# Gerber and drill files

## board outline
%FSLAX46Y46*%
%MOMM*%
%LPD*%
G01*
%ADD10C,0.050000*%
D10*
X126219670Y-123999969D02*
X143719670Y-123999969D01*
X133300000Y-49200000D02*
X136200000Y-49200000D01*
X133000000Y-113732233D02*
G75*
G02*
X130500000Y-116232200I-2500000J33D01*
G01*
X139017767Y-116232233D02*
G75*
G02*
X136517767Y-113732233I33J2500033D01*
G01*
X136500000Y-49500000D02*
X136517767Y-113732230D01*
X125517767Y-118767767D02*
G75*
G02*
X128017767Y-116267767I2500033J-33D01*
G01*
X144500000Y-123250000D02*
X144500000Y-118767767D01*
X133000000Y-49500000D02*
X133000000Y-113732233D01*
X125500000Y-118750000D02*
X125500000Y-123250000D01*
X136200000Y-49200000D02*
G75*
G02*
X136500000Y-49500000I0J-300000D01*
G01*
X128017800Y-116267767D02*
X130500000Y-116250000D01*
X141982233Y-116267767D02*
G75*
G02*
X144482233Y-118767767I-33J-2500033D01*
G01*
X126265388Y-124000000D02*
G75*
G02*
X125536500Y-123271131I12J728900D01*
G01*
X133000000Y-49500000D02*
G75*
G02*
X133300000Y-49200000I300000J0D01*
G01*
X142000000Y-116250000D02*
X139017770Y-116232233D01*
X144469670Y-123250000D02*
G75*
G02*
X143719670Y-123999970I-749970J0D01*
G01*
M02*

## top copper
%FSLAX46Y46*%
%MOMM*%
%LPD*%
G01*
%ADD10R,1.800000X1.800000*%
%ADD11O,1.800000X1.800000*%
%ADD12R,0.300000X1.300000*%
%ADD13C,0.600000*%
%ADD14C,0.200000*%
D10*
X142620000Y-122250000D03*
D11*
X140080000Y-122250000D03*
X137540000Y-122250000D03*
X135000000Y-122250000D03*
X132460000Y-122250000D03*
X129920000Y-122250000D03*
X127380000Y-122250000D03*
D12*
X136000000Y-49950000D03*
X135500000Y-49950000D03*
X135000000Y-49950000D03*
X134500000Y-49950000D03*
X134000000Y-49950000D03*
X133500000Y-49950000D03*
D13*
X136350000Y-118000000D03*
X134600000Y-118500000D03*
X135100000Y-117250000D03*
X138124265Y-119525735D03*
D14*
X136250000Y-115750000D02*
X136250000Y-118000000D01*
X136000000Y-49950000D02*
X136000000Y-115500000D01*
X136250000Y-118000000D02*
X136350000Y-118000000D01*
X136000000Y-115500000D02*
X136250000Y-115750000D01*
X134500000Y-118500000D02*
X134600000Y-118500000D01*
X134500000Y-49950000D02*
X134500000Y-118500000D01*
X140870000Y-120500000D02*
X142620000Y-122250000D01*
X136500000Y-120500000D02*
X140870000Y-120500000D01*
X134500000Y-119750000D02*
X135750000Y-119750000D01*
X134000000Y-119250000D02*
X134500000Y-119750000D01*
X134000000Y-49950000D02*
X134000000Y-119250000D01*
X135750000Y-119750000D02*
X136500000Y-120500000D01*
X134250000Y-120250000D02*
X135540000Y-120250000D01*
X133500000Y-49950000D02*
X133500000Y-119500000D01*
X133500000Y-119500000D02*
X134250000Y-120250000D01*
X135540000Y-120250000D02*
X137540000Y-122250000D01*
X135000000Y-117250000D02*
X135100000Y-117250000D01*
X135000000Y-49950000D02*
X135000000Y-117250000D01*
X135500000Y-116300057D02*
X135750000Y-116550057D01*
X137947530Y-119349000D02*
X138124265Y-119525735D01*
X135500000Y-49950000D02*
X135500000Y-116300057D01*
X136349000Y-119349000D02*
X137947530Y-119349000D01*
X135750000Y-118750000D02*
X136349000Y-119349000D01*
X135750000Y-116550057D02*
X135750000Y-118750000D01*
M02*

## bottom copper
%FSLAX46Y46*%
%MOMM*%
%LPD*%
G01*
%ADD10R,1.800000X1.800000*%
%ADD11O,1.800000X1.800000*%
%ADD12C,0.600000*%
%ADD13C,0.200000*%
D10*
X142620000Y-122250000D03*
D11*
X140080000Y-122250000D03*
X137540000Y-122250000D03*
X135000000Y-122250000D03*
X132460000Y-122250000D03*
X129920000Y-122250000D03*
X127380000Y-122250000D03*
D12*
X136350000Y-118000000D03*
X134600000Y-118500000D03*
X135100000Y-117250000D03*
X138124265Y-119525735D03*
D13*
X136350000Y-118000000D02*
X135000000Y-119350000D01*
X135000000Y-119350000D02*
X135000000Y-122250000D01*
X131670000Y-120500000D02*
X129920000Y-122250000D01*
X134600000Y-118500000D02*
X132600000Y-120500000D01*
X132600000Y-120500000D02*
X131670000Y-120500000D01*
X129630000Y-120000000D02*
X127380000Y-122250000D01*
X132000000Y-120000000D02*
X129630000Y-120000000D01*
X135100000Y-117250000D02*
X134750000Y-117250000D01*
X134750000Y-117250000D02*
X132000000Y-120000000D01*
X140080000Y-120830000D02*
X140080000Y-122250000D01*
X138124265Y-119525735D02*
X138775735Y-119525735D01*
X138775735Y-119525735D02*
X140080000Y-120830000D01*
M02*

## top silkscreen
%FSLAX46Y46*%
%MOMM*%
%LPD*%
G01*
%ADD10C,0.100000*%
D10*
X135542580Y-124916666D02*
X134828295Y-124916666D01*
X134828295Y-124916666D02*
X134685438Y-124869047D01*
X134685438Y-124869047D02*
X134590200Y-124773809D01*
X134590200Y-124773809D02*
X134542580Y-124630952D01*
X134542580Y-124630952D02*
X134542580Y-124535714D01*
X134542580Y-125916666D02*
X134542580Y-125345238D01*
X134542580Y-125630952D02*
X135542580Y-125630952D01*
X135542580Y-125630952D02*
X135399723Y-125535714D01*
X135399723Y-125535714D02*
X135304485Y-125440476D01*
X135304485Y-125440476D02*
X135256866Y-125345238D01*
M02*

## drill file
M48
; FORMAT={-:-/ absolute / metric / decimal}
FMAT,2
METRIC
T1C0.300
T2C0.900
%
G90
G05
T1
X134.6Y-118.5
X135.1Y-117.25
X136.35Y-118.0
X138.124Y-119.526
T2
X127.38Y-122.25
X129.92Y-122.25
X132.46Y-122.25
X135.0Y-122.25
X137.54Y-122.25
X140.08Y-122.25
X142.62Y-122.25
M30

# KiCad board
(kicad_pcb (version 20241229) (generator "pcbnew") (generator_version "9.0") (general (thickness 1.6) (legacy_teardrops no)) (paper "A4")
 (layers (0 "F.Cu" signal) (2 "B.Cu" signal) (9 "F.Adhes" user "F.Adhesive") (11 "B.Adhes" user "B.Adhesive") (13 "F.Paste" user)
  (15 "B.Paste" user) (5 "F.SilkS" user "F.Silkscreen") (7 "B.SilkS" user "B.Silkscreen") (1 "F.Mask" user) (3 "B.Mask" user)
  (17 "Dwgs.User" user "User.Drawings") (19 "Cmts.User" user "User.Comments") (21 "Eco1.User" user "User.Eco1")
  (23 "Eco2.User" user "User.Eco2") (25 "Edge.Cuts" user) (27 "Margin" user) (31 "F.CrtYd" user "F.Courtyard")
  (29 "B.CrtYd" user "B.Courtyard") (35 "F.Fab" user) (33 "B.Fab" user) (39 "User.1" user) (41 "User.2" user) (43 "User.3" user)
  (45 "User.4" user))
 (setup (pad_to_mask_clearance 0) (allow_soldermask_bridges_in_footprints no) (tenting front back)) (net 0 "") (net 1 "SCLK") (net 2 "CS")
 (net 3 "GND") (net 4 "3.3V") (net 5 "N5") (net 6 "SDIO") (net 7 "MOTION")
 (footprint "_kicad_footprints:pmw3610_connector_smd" (layer "F.Cu") (at 135 122.25 -90)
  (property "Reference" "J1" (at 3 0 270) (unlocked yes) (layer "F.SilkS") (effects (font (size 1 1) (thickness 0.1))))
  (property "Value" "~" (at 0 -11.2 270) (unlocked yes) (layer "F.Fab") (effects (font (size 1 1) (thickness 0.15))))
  (pad "1" thru_hole rect (at 0 -7.62 270) (size 1.8 1.8) (drill 0.9) (layers "*.Cu" "*.Mask") (remove_unused_layers no) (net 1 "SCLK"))
  (pad "2" thru_hole oval (at 0 -5.08 270) (size 1.8 1.8) (drill 0.9) (layers "*.Cu" "*.Mask") (remove_unused_layers no) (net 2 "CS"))
  (pad "3" thru_hole oval (at 0 -2.54 270) (size 1.8 1.8) (drill 0.9) (layers "*.Cu" "*.Mask") (remove_unused_layers no) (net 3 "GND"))
  (pad "4" thru_hole oval (at 0 0 270) (size 1.8 1.8) (drill 0.9) (layers "*.Cu" "*.Mask") (remove_unused_layers no) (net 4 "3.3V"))
  (pad "5" thru_hole oval (at 0 2.54 270) (size 1.8 1.8) (drill 0.9) (layers "*.Cu" "*.Mask") (remove_unused_layers no) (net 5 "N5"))
  (pad "6" thru_hole oval (at 0 5.08 270) (size 1.8 1.8) (drill 0.9) (layers "*.Cu" "*.Mask") (remove_unused_layers no) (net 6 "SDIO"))
  (pad "7" thru_hole oval (at 0 7.62 270) (size 1.8 1.8) (drill 0.9) (layers "*.Cu" "*.Mask") (remove_unused_layers no) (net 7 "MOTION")))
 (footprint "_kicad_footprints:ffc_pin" (layer "B.Cu") (at 134.5 45.95)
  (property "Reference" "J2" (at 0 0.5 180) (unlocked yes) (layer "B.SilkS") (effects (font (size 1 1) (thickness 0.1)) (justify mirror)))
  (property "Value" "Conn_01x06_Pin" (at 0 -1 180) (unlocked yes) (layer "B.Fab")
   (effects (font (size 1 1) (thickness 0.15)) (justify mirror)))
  (pad "1" smd rect (at 1.5 4) (size 0.3 1.3) (layers "F.Cu" "F.Mask" "F.Paste") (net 4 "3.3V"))
  (pad "2" smd rect (at 1 4) (size 0.3 1.3) (layers "F.Cu" "F.Mask" "F.Paste") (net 2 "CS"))
  (pad "3" smd rect (at 0.5 4) (size 0.3 1.3) (layers "F.Cu" "F.Mask" "F.Paste") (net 7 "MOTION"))
  (pad "4" smd rect (at 0 4) (size 0.3 1.3) (layers "F.Cu" "F.Mask" "F.Paste") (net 6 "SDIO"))
  (pad "5" smd rect (at -0.5 4) (size 0.3 1.3) (layers "F.Cu" "F.Mask" "F.Paste") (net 1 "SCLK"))
  (pad "6" smd rect (at -1 4) (size 0.3 1.3) (layers "F.Cu" "F.Mask" "F.Paste") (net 3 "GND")))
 (gr_line (start 126.21967 123.999969) (end 143.71967 123.999969) (stroke (width 0.05) (type default)) (layer "Edge.Cuts"))
 (gr_line (start 133.3 49.2) (end 136.2 49.2) (stroke (width 0.05) (type default)) (layer "Edge.Cuts"))
 (gr_arc (start 133 113.732233) (mid 132.267767 115.5) (end 130.5 116.232233) (stroke (width 0.05) (type default)) (layer "Edge.Cuts"))
 (gr_arc (start 139.017767 116.232233) (mid 137.25 115.5) (end 136.517767 113.732233) (stroke (width 0.05) (type default))
  (layer "Edge.Cuts"))
 (gr_line (start 136.5 49.5) (end 136.517767 113.73223) (stroke (width 0.05) (type default)) (layer "Edge.Cuts"))
 (gr_arc (start 125.517767 118.767767) (mid 126.25 117) (end 128.017767 116.267767) (stroke (width 0.05) (type default)) (layer "Edge.Cuts"))
 (gr_line (start 144.5 123.25) (end 144.5 118.767767) (stroke (width 0.05) (type default)) (layer "Edge.Cuts"))
 (gr_line (start 133 49.5) (end 133 113.732233) (stroke (width 0.05) (type default)) (layer "Edge.Cuts"))
 (gr_line (start 125.5 118.75) (end 125.5 123.25) (stroke (width 0.05) (type default)) (layer "Edge.Cuts"))
 (gr_arc (start 136.2 49.2) (mid 136.412132 49.287868) (end 136.5 49.5) (stroke (width 0.05) (type default)) (layer "Edge.Cuts"))
 (gr_line (start 128.0178 116.267767) (end 130.5 116.25) (stroke (width 0.05) (type default)) (layer "Edge.Cuts"))
 (gr_arc (start 141.982233 116.267767) (mid 143.75 117) (end 144.482233 118.767767) (stroke (width 0.05) (type default)) (layer "Edge.Cuts"))
 (gr_arc (start 126.265388 124) (mid 125.75 123.786519) (end 125.536519 123.271131) (stroke (width 0.05) (type default)) (layer "Edge.Cuts"))
 (gr_arc (start 133 49.5) (mid 133.087868 49.287868) (end 133.3 49.2) (stroke (width 0.05) (type default)) (layer "Edge.Cuts"))
 (gr_line (start 142 116.25) (end 139.01777 116.232233) (stroke (width 0.05) (type default)) (layer "Edge.Cuts"))
 (gr_arc (start 144.46967 123.25) (mid 144.25 123.78033) (end 143.71967 124) (stroke (width 0.05) (type default)) (layer "Edge.Cuts"))
 (segment (start 136.25 115.75) (end 136.25 118) (width 0.2) (layer "F.Cu") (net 4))
 (segment (start 136 49.95) (end 136 115.5) (width 0.2) (layer "F.Cu") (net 4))
 (segment (start 136.25 118) (end 136.35 118) (width 0.2) (layer "F.Cu") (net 4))
 (segment (start 136 115.5) (end 136.25 115.75) (width 0.2) (layer "F.Cu") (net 4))
 (via (at 136.35 118) (size 0.6) (drill 0.3) (layers "F.Cu" "B.Cu") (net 4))
 (segment (start 136.35 118) (end 135 119.35) (width 0.2) (layer "B.Cu") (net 4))
 (segment (start 135 119.35) (end 135 122.25) (width 0.2) (layer "B.Cu") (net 4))
 (segment (start 134.5 118.5) (end 134.6 118.5) (width 0.2) (layer "F.Cu") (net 6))
 (segment (start 134.5 49.95) (end 134.5 118.5) (width 0.2) (layer "F.Cu") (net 6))
 (via (at 134.6 118.5) (size 0.6) (drill 0.3) (layers "F.Cu" "B.Cu") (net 6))
 (segment (start 131.67 120.5) (end 129.92 122.25) (width 0.2) (layer "B.Cu") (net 6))
 (segment (start 134.6 118.5) (end 132.6 120.5) (width 0.2) (layer "B.Cu") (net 6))
 (segment (start 132.6 120.5) (end 131.67 120.5) (width 0.2) (layer "B.Cu") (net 6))
 (segment (start 140.87 120.5) (end 142.62 122.25) (width 0.2) (layer "F.Cu") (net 1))
 (segment (start 136.5 120.5) (end 140.87 120.5) (width 0.2) (layer "F.Cu") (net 1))
 (segment (start 134.5 119.75) (end 135.75 119.75) (width 0.2) (layer "F.Cu") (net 1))
 (segment (start 134 119.25) (end 134.5 119.75) (width 0.2) (layer "F.Cu") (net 1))
 (segment (start 134 49.95) (end 134 119.25) (width 0.2) (layer "F.Cu") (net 1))
 (segment (start 135.75 119.75) (end 136.5 120.5) (width 0.2) (layer "F.Cu") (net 1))
 (segment (start 134.25 120.25) (end 135.54 120.25) (width 0.2) (layer "F.Cu") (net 3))
 (segment (start 133.5 49.95) (end 133.5 119.5) (width 0.2) (layer "F.Cu") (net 3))
 (segment (start 133.5 119.5) (end 134.25 120.25) (width 0.2) (layer "F.Cu") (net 3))
 (segment (start 135.54 120.25) (end 137.54 122.25) (width 0.2) (layer "F.Cu") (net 3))
 (segment (start 135 117.25) (end 135.1 117.25) (width 0.2) (layer "F.Cu") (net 7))
 (segment (start 135 49.95) (end 135 117.25) (width 0.2) (layer "F.Cu") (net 7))
 (via (at 135.1 117.25) (size 0.6) (drill 0.3) (layers "F.Cu" "B.Cu") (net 7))
 (segment (start 129.63 120) (end 127.38 122.25) (width 0.2) (layer "B.Cu") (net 7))
 (segment (start 132 120) (end 129.63 120) (width 0.2) (layer "B.Cu") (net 7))
 (segment (start 135.1 117.25) (end 134.75 117.25) (width 0.2) (layer "B.Cu") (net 7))
 (segment (start 134.75 117.25) (end 132 120) (width 0.2) (layer "B.Cu") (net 7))
 (segment (start 135.5 116.300057) (end 135.75 116.550057) (width 0.2) (layer "F.Cu") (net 2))
 (segment (start 137.94753 119.349) (end 138.124265 119.525735) (width 0.2) (layer "F.Cu") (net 2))
 (segment (start 135.5 49.95) (end 135.5 116.300057) (width 0.2) (layer "F.Cu") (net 2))
 (segment (start 136.349 119.349) (end 137.94753 119.349) (width 0.2) (layer "F.Cu") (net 2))
 (segment (start 135.75 118.75) (end 136.349 119.349) (width 0.2) (layer "F.Cu") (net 2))
 (segment (start 135.75 116.550057) (end 135.75 118.75) (width 0.2) (layer "F.Cu") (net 2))
 (via (at 138.124265 119.525735) (size 0.6) (drill 0.3) (layers "F.Cu" "B.Cu") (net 2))
 (segment (start 140.08 120.83) (end 140.08 122.25) (width 0.2) (layer "B.Cu") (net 2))
 (segment (start 138.124265 119.525735) (end 138.775735 119.525735) (width 0.2) (layer "B.Cu") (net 2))
 (segment (start 138.775735 119.525735) (end 140.08 120.83) (width 0.2) (layer "B.Cu") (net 2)))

